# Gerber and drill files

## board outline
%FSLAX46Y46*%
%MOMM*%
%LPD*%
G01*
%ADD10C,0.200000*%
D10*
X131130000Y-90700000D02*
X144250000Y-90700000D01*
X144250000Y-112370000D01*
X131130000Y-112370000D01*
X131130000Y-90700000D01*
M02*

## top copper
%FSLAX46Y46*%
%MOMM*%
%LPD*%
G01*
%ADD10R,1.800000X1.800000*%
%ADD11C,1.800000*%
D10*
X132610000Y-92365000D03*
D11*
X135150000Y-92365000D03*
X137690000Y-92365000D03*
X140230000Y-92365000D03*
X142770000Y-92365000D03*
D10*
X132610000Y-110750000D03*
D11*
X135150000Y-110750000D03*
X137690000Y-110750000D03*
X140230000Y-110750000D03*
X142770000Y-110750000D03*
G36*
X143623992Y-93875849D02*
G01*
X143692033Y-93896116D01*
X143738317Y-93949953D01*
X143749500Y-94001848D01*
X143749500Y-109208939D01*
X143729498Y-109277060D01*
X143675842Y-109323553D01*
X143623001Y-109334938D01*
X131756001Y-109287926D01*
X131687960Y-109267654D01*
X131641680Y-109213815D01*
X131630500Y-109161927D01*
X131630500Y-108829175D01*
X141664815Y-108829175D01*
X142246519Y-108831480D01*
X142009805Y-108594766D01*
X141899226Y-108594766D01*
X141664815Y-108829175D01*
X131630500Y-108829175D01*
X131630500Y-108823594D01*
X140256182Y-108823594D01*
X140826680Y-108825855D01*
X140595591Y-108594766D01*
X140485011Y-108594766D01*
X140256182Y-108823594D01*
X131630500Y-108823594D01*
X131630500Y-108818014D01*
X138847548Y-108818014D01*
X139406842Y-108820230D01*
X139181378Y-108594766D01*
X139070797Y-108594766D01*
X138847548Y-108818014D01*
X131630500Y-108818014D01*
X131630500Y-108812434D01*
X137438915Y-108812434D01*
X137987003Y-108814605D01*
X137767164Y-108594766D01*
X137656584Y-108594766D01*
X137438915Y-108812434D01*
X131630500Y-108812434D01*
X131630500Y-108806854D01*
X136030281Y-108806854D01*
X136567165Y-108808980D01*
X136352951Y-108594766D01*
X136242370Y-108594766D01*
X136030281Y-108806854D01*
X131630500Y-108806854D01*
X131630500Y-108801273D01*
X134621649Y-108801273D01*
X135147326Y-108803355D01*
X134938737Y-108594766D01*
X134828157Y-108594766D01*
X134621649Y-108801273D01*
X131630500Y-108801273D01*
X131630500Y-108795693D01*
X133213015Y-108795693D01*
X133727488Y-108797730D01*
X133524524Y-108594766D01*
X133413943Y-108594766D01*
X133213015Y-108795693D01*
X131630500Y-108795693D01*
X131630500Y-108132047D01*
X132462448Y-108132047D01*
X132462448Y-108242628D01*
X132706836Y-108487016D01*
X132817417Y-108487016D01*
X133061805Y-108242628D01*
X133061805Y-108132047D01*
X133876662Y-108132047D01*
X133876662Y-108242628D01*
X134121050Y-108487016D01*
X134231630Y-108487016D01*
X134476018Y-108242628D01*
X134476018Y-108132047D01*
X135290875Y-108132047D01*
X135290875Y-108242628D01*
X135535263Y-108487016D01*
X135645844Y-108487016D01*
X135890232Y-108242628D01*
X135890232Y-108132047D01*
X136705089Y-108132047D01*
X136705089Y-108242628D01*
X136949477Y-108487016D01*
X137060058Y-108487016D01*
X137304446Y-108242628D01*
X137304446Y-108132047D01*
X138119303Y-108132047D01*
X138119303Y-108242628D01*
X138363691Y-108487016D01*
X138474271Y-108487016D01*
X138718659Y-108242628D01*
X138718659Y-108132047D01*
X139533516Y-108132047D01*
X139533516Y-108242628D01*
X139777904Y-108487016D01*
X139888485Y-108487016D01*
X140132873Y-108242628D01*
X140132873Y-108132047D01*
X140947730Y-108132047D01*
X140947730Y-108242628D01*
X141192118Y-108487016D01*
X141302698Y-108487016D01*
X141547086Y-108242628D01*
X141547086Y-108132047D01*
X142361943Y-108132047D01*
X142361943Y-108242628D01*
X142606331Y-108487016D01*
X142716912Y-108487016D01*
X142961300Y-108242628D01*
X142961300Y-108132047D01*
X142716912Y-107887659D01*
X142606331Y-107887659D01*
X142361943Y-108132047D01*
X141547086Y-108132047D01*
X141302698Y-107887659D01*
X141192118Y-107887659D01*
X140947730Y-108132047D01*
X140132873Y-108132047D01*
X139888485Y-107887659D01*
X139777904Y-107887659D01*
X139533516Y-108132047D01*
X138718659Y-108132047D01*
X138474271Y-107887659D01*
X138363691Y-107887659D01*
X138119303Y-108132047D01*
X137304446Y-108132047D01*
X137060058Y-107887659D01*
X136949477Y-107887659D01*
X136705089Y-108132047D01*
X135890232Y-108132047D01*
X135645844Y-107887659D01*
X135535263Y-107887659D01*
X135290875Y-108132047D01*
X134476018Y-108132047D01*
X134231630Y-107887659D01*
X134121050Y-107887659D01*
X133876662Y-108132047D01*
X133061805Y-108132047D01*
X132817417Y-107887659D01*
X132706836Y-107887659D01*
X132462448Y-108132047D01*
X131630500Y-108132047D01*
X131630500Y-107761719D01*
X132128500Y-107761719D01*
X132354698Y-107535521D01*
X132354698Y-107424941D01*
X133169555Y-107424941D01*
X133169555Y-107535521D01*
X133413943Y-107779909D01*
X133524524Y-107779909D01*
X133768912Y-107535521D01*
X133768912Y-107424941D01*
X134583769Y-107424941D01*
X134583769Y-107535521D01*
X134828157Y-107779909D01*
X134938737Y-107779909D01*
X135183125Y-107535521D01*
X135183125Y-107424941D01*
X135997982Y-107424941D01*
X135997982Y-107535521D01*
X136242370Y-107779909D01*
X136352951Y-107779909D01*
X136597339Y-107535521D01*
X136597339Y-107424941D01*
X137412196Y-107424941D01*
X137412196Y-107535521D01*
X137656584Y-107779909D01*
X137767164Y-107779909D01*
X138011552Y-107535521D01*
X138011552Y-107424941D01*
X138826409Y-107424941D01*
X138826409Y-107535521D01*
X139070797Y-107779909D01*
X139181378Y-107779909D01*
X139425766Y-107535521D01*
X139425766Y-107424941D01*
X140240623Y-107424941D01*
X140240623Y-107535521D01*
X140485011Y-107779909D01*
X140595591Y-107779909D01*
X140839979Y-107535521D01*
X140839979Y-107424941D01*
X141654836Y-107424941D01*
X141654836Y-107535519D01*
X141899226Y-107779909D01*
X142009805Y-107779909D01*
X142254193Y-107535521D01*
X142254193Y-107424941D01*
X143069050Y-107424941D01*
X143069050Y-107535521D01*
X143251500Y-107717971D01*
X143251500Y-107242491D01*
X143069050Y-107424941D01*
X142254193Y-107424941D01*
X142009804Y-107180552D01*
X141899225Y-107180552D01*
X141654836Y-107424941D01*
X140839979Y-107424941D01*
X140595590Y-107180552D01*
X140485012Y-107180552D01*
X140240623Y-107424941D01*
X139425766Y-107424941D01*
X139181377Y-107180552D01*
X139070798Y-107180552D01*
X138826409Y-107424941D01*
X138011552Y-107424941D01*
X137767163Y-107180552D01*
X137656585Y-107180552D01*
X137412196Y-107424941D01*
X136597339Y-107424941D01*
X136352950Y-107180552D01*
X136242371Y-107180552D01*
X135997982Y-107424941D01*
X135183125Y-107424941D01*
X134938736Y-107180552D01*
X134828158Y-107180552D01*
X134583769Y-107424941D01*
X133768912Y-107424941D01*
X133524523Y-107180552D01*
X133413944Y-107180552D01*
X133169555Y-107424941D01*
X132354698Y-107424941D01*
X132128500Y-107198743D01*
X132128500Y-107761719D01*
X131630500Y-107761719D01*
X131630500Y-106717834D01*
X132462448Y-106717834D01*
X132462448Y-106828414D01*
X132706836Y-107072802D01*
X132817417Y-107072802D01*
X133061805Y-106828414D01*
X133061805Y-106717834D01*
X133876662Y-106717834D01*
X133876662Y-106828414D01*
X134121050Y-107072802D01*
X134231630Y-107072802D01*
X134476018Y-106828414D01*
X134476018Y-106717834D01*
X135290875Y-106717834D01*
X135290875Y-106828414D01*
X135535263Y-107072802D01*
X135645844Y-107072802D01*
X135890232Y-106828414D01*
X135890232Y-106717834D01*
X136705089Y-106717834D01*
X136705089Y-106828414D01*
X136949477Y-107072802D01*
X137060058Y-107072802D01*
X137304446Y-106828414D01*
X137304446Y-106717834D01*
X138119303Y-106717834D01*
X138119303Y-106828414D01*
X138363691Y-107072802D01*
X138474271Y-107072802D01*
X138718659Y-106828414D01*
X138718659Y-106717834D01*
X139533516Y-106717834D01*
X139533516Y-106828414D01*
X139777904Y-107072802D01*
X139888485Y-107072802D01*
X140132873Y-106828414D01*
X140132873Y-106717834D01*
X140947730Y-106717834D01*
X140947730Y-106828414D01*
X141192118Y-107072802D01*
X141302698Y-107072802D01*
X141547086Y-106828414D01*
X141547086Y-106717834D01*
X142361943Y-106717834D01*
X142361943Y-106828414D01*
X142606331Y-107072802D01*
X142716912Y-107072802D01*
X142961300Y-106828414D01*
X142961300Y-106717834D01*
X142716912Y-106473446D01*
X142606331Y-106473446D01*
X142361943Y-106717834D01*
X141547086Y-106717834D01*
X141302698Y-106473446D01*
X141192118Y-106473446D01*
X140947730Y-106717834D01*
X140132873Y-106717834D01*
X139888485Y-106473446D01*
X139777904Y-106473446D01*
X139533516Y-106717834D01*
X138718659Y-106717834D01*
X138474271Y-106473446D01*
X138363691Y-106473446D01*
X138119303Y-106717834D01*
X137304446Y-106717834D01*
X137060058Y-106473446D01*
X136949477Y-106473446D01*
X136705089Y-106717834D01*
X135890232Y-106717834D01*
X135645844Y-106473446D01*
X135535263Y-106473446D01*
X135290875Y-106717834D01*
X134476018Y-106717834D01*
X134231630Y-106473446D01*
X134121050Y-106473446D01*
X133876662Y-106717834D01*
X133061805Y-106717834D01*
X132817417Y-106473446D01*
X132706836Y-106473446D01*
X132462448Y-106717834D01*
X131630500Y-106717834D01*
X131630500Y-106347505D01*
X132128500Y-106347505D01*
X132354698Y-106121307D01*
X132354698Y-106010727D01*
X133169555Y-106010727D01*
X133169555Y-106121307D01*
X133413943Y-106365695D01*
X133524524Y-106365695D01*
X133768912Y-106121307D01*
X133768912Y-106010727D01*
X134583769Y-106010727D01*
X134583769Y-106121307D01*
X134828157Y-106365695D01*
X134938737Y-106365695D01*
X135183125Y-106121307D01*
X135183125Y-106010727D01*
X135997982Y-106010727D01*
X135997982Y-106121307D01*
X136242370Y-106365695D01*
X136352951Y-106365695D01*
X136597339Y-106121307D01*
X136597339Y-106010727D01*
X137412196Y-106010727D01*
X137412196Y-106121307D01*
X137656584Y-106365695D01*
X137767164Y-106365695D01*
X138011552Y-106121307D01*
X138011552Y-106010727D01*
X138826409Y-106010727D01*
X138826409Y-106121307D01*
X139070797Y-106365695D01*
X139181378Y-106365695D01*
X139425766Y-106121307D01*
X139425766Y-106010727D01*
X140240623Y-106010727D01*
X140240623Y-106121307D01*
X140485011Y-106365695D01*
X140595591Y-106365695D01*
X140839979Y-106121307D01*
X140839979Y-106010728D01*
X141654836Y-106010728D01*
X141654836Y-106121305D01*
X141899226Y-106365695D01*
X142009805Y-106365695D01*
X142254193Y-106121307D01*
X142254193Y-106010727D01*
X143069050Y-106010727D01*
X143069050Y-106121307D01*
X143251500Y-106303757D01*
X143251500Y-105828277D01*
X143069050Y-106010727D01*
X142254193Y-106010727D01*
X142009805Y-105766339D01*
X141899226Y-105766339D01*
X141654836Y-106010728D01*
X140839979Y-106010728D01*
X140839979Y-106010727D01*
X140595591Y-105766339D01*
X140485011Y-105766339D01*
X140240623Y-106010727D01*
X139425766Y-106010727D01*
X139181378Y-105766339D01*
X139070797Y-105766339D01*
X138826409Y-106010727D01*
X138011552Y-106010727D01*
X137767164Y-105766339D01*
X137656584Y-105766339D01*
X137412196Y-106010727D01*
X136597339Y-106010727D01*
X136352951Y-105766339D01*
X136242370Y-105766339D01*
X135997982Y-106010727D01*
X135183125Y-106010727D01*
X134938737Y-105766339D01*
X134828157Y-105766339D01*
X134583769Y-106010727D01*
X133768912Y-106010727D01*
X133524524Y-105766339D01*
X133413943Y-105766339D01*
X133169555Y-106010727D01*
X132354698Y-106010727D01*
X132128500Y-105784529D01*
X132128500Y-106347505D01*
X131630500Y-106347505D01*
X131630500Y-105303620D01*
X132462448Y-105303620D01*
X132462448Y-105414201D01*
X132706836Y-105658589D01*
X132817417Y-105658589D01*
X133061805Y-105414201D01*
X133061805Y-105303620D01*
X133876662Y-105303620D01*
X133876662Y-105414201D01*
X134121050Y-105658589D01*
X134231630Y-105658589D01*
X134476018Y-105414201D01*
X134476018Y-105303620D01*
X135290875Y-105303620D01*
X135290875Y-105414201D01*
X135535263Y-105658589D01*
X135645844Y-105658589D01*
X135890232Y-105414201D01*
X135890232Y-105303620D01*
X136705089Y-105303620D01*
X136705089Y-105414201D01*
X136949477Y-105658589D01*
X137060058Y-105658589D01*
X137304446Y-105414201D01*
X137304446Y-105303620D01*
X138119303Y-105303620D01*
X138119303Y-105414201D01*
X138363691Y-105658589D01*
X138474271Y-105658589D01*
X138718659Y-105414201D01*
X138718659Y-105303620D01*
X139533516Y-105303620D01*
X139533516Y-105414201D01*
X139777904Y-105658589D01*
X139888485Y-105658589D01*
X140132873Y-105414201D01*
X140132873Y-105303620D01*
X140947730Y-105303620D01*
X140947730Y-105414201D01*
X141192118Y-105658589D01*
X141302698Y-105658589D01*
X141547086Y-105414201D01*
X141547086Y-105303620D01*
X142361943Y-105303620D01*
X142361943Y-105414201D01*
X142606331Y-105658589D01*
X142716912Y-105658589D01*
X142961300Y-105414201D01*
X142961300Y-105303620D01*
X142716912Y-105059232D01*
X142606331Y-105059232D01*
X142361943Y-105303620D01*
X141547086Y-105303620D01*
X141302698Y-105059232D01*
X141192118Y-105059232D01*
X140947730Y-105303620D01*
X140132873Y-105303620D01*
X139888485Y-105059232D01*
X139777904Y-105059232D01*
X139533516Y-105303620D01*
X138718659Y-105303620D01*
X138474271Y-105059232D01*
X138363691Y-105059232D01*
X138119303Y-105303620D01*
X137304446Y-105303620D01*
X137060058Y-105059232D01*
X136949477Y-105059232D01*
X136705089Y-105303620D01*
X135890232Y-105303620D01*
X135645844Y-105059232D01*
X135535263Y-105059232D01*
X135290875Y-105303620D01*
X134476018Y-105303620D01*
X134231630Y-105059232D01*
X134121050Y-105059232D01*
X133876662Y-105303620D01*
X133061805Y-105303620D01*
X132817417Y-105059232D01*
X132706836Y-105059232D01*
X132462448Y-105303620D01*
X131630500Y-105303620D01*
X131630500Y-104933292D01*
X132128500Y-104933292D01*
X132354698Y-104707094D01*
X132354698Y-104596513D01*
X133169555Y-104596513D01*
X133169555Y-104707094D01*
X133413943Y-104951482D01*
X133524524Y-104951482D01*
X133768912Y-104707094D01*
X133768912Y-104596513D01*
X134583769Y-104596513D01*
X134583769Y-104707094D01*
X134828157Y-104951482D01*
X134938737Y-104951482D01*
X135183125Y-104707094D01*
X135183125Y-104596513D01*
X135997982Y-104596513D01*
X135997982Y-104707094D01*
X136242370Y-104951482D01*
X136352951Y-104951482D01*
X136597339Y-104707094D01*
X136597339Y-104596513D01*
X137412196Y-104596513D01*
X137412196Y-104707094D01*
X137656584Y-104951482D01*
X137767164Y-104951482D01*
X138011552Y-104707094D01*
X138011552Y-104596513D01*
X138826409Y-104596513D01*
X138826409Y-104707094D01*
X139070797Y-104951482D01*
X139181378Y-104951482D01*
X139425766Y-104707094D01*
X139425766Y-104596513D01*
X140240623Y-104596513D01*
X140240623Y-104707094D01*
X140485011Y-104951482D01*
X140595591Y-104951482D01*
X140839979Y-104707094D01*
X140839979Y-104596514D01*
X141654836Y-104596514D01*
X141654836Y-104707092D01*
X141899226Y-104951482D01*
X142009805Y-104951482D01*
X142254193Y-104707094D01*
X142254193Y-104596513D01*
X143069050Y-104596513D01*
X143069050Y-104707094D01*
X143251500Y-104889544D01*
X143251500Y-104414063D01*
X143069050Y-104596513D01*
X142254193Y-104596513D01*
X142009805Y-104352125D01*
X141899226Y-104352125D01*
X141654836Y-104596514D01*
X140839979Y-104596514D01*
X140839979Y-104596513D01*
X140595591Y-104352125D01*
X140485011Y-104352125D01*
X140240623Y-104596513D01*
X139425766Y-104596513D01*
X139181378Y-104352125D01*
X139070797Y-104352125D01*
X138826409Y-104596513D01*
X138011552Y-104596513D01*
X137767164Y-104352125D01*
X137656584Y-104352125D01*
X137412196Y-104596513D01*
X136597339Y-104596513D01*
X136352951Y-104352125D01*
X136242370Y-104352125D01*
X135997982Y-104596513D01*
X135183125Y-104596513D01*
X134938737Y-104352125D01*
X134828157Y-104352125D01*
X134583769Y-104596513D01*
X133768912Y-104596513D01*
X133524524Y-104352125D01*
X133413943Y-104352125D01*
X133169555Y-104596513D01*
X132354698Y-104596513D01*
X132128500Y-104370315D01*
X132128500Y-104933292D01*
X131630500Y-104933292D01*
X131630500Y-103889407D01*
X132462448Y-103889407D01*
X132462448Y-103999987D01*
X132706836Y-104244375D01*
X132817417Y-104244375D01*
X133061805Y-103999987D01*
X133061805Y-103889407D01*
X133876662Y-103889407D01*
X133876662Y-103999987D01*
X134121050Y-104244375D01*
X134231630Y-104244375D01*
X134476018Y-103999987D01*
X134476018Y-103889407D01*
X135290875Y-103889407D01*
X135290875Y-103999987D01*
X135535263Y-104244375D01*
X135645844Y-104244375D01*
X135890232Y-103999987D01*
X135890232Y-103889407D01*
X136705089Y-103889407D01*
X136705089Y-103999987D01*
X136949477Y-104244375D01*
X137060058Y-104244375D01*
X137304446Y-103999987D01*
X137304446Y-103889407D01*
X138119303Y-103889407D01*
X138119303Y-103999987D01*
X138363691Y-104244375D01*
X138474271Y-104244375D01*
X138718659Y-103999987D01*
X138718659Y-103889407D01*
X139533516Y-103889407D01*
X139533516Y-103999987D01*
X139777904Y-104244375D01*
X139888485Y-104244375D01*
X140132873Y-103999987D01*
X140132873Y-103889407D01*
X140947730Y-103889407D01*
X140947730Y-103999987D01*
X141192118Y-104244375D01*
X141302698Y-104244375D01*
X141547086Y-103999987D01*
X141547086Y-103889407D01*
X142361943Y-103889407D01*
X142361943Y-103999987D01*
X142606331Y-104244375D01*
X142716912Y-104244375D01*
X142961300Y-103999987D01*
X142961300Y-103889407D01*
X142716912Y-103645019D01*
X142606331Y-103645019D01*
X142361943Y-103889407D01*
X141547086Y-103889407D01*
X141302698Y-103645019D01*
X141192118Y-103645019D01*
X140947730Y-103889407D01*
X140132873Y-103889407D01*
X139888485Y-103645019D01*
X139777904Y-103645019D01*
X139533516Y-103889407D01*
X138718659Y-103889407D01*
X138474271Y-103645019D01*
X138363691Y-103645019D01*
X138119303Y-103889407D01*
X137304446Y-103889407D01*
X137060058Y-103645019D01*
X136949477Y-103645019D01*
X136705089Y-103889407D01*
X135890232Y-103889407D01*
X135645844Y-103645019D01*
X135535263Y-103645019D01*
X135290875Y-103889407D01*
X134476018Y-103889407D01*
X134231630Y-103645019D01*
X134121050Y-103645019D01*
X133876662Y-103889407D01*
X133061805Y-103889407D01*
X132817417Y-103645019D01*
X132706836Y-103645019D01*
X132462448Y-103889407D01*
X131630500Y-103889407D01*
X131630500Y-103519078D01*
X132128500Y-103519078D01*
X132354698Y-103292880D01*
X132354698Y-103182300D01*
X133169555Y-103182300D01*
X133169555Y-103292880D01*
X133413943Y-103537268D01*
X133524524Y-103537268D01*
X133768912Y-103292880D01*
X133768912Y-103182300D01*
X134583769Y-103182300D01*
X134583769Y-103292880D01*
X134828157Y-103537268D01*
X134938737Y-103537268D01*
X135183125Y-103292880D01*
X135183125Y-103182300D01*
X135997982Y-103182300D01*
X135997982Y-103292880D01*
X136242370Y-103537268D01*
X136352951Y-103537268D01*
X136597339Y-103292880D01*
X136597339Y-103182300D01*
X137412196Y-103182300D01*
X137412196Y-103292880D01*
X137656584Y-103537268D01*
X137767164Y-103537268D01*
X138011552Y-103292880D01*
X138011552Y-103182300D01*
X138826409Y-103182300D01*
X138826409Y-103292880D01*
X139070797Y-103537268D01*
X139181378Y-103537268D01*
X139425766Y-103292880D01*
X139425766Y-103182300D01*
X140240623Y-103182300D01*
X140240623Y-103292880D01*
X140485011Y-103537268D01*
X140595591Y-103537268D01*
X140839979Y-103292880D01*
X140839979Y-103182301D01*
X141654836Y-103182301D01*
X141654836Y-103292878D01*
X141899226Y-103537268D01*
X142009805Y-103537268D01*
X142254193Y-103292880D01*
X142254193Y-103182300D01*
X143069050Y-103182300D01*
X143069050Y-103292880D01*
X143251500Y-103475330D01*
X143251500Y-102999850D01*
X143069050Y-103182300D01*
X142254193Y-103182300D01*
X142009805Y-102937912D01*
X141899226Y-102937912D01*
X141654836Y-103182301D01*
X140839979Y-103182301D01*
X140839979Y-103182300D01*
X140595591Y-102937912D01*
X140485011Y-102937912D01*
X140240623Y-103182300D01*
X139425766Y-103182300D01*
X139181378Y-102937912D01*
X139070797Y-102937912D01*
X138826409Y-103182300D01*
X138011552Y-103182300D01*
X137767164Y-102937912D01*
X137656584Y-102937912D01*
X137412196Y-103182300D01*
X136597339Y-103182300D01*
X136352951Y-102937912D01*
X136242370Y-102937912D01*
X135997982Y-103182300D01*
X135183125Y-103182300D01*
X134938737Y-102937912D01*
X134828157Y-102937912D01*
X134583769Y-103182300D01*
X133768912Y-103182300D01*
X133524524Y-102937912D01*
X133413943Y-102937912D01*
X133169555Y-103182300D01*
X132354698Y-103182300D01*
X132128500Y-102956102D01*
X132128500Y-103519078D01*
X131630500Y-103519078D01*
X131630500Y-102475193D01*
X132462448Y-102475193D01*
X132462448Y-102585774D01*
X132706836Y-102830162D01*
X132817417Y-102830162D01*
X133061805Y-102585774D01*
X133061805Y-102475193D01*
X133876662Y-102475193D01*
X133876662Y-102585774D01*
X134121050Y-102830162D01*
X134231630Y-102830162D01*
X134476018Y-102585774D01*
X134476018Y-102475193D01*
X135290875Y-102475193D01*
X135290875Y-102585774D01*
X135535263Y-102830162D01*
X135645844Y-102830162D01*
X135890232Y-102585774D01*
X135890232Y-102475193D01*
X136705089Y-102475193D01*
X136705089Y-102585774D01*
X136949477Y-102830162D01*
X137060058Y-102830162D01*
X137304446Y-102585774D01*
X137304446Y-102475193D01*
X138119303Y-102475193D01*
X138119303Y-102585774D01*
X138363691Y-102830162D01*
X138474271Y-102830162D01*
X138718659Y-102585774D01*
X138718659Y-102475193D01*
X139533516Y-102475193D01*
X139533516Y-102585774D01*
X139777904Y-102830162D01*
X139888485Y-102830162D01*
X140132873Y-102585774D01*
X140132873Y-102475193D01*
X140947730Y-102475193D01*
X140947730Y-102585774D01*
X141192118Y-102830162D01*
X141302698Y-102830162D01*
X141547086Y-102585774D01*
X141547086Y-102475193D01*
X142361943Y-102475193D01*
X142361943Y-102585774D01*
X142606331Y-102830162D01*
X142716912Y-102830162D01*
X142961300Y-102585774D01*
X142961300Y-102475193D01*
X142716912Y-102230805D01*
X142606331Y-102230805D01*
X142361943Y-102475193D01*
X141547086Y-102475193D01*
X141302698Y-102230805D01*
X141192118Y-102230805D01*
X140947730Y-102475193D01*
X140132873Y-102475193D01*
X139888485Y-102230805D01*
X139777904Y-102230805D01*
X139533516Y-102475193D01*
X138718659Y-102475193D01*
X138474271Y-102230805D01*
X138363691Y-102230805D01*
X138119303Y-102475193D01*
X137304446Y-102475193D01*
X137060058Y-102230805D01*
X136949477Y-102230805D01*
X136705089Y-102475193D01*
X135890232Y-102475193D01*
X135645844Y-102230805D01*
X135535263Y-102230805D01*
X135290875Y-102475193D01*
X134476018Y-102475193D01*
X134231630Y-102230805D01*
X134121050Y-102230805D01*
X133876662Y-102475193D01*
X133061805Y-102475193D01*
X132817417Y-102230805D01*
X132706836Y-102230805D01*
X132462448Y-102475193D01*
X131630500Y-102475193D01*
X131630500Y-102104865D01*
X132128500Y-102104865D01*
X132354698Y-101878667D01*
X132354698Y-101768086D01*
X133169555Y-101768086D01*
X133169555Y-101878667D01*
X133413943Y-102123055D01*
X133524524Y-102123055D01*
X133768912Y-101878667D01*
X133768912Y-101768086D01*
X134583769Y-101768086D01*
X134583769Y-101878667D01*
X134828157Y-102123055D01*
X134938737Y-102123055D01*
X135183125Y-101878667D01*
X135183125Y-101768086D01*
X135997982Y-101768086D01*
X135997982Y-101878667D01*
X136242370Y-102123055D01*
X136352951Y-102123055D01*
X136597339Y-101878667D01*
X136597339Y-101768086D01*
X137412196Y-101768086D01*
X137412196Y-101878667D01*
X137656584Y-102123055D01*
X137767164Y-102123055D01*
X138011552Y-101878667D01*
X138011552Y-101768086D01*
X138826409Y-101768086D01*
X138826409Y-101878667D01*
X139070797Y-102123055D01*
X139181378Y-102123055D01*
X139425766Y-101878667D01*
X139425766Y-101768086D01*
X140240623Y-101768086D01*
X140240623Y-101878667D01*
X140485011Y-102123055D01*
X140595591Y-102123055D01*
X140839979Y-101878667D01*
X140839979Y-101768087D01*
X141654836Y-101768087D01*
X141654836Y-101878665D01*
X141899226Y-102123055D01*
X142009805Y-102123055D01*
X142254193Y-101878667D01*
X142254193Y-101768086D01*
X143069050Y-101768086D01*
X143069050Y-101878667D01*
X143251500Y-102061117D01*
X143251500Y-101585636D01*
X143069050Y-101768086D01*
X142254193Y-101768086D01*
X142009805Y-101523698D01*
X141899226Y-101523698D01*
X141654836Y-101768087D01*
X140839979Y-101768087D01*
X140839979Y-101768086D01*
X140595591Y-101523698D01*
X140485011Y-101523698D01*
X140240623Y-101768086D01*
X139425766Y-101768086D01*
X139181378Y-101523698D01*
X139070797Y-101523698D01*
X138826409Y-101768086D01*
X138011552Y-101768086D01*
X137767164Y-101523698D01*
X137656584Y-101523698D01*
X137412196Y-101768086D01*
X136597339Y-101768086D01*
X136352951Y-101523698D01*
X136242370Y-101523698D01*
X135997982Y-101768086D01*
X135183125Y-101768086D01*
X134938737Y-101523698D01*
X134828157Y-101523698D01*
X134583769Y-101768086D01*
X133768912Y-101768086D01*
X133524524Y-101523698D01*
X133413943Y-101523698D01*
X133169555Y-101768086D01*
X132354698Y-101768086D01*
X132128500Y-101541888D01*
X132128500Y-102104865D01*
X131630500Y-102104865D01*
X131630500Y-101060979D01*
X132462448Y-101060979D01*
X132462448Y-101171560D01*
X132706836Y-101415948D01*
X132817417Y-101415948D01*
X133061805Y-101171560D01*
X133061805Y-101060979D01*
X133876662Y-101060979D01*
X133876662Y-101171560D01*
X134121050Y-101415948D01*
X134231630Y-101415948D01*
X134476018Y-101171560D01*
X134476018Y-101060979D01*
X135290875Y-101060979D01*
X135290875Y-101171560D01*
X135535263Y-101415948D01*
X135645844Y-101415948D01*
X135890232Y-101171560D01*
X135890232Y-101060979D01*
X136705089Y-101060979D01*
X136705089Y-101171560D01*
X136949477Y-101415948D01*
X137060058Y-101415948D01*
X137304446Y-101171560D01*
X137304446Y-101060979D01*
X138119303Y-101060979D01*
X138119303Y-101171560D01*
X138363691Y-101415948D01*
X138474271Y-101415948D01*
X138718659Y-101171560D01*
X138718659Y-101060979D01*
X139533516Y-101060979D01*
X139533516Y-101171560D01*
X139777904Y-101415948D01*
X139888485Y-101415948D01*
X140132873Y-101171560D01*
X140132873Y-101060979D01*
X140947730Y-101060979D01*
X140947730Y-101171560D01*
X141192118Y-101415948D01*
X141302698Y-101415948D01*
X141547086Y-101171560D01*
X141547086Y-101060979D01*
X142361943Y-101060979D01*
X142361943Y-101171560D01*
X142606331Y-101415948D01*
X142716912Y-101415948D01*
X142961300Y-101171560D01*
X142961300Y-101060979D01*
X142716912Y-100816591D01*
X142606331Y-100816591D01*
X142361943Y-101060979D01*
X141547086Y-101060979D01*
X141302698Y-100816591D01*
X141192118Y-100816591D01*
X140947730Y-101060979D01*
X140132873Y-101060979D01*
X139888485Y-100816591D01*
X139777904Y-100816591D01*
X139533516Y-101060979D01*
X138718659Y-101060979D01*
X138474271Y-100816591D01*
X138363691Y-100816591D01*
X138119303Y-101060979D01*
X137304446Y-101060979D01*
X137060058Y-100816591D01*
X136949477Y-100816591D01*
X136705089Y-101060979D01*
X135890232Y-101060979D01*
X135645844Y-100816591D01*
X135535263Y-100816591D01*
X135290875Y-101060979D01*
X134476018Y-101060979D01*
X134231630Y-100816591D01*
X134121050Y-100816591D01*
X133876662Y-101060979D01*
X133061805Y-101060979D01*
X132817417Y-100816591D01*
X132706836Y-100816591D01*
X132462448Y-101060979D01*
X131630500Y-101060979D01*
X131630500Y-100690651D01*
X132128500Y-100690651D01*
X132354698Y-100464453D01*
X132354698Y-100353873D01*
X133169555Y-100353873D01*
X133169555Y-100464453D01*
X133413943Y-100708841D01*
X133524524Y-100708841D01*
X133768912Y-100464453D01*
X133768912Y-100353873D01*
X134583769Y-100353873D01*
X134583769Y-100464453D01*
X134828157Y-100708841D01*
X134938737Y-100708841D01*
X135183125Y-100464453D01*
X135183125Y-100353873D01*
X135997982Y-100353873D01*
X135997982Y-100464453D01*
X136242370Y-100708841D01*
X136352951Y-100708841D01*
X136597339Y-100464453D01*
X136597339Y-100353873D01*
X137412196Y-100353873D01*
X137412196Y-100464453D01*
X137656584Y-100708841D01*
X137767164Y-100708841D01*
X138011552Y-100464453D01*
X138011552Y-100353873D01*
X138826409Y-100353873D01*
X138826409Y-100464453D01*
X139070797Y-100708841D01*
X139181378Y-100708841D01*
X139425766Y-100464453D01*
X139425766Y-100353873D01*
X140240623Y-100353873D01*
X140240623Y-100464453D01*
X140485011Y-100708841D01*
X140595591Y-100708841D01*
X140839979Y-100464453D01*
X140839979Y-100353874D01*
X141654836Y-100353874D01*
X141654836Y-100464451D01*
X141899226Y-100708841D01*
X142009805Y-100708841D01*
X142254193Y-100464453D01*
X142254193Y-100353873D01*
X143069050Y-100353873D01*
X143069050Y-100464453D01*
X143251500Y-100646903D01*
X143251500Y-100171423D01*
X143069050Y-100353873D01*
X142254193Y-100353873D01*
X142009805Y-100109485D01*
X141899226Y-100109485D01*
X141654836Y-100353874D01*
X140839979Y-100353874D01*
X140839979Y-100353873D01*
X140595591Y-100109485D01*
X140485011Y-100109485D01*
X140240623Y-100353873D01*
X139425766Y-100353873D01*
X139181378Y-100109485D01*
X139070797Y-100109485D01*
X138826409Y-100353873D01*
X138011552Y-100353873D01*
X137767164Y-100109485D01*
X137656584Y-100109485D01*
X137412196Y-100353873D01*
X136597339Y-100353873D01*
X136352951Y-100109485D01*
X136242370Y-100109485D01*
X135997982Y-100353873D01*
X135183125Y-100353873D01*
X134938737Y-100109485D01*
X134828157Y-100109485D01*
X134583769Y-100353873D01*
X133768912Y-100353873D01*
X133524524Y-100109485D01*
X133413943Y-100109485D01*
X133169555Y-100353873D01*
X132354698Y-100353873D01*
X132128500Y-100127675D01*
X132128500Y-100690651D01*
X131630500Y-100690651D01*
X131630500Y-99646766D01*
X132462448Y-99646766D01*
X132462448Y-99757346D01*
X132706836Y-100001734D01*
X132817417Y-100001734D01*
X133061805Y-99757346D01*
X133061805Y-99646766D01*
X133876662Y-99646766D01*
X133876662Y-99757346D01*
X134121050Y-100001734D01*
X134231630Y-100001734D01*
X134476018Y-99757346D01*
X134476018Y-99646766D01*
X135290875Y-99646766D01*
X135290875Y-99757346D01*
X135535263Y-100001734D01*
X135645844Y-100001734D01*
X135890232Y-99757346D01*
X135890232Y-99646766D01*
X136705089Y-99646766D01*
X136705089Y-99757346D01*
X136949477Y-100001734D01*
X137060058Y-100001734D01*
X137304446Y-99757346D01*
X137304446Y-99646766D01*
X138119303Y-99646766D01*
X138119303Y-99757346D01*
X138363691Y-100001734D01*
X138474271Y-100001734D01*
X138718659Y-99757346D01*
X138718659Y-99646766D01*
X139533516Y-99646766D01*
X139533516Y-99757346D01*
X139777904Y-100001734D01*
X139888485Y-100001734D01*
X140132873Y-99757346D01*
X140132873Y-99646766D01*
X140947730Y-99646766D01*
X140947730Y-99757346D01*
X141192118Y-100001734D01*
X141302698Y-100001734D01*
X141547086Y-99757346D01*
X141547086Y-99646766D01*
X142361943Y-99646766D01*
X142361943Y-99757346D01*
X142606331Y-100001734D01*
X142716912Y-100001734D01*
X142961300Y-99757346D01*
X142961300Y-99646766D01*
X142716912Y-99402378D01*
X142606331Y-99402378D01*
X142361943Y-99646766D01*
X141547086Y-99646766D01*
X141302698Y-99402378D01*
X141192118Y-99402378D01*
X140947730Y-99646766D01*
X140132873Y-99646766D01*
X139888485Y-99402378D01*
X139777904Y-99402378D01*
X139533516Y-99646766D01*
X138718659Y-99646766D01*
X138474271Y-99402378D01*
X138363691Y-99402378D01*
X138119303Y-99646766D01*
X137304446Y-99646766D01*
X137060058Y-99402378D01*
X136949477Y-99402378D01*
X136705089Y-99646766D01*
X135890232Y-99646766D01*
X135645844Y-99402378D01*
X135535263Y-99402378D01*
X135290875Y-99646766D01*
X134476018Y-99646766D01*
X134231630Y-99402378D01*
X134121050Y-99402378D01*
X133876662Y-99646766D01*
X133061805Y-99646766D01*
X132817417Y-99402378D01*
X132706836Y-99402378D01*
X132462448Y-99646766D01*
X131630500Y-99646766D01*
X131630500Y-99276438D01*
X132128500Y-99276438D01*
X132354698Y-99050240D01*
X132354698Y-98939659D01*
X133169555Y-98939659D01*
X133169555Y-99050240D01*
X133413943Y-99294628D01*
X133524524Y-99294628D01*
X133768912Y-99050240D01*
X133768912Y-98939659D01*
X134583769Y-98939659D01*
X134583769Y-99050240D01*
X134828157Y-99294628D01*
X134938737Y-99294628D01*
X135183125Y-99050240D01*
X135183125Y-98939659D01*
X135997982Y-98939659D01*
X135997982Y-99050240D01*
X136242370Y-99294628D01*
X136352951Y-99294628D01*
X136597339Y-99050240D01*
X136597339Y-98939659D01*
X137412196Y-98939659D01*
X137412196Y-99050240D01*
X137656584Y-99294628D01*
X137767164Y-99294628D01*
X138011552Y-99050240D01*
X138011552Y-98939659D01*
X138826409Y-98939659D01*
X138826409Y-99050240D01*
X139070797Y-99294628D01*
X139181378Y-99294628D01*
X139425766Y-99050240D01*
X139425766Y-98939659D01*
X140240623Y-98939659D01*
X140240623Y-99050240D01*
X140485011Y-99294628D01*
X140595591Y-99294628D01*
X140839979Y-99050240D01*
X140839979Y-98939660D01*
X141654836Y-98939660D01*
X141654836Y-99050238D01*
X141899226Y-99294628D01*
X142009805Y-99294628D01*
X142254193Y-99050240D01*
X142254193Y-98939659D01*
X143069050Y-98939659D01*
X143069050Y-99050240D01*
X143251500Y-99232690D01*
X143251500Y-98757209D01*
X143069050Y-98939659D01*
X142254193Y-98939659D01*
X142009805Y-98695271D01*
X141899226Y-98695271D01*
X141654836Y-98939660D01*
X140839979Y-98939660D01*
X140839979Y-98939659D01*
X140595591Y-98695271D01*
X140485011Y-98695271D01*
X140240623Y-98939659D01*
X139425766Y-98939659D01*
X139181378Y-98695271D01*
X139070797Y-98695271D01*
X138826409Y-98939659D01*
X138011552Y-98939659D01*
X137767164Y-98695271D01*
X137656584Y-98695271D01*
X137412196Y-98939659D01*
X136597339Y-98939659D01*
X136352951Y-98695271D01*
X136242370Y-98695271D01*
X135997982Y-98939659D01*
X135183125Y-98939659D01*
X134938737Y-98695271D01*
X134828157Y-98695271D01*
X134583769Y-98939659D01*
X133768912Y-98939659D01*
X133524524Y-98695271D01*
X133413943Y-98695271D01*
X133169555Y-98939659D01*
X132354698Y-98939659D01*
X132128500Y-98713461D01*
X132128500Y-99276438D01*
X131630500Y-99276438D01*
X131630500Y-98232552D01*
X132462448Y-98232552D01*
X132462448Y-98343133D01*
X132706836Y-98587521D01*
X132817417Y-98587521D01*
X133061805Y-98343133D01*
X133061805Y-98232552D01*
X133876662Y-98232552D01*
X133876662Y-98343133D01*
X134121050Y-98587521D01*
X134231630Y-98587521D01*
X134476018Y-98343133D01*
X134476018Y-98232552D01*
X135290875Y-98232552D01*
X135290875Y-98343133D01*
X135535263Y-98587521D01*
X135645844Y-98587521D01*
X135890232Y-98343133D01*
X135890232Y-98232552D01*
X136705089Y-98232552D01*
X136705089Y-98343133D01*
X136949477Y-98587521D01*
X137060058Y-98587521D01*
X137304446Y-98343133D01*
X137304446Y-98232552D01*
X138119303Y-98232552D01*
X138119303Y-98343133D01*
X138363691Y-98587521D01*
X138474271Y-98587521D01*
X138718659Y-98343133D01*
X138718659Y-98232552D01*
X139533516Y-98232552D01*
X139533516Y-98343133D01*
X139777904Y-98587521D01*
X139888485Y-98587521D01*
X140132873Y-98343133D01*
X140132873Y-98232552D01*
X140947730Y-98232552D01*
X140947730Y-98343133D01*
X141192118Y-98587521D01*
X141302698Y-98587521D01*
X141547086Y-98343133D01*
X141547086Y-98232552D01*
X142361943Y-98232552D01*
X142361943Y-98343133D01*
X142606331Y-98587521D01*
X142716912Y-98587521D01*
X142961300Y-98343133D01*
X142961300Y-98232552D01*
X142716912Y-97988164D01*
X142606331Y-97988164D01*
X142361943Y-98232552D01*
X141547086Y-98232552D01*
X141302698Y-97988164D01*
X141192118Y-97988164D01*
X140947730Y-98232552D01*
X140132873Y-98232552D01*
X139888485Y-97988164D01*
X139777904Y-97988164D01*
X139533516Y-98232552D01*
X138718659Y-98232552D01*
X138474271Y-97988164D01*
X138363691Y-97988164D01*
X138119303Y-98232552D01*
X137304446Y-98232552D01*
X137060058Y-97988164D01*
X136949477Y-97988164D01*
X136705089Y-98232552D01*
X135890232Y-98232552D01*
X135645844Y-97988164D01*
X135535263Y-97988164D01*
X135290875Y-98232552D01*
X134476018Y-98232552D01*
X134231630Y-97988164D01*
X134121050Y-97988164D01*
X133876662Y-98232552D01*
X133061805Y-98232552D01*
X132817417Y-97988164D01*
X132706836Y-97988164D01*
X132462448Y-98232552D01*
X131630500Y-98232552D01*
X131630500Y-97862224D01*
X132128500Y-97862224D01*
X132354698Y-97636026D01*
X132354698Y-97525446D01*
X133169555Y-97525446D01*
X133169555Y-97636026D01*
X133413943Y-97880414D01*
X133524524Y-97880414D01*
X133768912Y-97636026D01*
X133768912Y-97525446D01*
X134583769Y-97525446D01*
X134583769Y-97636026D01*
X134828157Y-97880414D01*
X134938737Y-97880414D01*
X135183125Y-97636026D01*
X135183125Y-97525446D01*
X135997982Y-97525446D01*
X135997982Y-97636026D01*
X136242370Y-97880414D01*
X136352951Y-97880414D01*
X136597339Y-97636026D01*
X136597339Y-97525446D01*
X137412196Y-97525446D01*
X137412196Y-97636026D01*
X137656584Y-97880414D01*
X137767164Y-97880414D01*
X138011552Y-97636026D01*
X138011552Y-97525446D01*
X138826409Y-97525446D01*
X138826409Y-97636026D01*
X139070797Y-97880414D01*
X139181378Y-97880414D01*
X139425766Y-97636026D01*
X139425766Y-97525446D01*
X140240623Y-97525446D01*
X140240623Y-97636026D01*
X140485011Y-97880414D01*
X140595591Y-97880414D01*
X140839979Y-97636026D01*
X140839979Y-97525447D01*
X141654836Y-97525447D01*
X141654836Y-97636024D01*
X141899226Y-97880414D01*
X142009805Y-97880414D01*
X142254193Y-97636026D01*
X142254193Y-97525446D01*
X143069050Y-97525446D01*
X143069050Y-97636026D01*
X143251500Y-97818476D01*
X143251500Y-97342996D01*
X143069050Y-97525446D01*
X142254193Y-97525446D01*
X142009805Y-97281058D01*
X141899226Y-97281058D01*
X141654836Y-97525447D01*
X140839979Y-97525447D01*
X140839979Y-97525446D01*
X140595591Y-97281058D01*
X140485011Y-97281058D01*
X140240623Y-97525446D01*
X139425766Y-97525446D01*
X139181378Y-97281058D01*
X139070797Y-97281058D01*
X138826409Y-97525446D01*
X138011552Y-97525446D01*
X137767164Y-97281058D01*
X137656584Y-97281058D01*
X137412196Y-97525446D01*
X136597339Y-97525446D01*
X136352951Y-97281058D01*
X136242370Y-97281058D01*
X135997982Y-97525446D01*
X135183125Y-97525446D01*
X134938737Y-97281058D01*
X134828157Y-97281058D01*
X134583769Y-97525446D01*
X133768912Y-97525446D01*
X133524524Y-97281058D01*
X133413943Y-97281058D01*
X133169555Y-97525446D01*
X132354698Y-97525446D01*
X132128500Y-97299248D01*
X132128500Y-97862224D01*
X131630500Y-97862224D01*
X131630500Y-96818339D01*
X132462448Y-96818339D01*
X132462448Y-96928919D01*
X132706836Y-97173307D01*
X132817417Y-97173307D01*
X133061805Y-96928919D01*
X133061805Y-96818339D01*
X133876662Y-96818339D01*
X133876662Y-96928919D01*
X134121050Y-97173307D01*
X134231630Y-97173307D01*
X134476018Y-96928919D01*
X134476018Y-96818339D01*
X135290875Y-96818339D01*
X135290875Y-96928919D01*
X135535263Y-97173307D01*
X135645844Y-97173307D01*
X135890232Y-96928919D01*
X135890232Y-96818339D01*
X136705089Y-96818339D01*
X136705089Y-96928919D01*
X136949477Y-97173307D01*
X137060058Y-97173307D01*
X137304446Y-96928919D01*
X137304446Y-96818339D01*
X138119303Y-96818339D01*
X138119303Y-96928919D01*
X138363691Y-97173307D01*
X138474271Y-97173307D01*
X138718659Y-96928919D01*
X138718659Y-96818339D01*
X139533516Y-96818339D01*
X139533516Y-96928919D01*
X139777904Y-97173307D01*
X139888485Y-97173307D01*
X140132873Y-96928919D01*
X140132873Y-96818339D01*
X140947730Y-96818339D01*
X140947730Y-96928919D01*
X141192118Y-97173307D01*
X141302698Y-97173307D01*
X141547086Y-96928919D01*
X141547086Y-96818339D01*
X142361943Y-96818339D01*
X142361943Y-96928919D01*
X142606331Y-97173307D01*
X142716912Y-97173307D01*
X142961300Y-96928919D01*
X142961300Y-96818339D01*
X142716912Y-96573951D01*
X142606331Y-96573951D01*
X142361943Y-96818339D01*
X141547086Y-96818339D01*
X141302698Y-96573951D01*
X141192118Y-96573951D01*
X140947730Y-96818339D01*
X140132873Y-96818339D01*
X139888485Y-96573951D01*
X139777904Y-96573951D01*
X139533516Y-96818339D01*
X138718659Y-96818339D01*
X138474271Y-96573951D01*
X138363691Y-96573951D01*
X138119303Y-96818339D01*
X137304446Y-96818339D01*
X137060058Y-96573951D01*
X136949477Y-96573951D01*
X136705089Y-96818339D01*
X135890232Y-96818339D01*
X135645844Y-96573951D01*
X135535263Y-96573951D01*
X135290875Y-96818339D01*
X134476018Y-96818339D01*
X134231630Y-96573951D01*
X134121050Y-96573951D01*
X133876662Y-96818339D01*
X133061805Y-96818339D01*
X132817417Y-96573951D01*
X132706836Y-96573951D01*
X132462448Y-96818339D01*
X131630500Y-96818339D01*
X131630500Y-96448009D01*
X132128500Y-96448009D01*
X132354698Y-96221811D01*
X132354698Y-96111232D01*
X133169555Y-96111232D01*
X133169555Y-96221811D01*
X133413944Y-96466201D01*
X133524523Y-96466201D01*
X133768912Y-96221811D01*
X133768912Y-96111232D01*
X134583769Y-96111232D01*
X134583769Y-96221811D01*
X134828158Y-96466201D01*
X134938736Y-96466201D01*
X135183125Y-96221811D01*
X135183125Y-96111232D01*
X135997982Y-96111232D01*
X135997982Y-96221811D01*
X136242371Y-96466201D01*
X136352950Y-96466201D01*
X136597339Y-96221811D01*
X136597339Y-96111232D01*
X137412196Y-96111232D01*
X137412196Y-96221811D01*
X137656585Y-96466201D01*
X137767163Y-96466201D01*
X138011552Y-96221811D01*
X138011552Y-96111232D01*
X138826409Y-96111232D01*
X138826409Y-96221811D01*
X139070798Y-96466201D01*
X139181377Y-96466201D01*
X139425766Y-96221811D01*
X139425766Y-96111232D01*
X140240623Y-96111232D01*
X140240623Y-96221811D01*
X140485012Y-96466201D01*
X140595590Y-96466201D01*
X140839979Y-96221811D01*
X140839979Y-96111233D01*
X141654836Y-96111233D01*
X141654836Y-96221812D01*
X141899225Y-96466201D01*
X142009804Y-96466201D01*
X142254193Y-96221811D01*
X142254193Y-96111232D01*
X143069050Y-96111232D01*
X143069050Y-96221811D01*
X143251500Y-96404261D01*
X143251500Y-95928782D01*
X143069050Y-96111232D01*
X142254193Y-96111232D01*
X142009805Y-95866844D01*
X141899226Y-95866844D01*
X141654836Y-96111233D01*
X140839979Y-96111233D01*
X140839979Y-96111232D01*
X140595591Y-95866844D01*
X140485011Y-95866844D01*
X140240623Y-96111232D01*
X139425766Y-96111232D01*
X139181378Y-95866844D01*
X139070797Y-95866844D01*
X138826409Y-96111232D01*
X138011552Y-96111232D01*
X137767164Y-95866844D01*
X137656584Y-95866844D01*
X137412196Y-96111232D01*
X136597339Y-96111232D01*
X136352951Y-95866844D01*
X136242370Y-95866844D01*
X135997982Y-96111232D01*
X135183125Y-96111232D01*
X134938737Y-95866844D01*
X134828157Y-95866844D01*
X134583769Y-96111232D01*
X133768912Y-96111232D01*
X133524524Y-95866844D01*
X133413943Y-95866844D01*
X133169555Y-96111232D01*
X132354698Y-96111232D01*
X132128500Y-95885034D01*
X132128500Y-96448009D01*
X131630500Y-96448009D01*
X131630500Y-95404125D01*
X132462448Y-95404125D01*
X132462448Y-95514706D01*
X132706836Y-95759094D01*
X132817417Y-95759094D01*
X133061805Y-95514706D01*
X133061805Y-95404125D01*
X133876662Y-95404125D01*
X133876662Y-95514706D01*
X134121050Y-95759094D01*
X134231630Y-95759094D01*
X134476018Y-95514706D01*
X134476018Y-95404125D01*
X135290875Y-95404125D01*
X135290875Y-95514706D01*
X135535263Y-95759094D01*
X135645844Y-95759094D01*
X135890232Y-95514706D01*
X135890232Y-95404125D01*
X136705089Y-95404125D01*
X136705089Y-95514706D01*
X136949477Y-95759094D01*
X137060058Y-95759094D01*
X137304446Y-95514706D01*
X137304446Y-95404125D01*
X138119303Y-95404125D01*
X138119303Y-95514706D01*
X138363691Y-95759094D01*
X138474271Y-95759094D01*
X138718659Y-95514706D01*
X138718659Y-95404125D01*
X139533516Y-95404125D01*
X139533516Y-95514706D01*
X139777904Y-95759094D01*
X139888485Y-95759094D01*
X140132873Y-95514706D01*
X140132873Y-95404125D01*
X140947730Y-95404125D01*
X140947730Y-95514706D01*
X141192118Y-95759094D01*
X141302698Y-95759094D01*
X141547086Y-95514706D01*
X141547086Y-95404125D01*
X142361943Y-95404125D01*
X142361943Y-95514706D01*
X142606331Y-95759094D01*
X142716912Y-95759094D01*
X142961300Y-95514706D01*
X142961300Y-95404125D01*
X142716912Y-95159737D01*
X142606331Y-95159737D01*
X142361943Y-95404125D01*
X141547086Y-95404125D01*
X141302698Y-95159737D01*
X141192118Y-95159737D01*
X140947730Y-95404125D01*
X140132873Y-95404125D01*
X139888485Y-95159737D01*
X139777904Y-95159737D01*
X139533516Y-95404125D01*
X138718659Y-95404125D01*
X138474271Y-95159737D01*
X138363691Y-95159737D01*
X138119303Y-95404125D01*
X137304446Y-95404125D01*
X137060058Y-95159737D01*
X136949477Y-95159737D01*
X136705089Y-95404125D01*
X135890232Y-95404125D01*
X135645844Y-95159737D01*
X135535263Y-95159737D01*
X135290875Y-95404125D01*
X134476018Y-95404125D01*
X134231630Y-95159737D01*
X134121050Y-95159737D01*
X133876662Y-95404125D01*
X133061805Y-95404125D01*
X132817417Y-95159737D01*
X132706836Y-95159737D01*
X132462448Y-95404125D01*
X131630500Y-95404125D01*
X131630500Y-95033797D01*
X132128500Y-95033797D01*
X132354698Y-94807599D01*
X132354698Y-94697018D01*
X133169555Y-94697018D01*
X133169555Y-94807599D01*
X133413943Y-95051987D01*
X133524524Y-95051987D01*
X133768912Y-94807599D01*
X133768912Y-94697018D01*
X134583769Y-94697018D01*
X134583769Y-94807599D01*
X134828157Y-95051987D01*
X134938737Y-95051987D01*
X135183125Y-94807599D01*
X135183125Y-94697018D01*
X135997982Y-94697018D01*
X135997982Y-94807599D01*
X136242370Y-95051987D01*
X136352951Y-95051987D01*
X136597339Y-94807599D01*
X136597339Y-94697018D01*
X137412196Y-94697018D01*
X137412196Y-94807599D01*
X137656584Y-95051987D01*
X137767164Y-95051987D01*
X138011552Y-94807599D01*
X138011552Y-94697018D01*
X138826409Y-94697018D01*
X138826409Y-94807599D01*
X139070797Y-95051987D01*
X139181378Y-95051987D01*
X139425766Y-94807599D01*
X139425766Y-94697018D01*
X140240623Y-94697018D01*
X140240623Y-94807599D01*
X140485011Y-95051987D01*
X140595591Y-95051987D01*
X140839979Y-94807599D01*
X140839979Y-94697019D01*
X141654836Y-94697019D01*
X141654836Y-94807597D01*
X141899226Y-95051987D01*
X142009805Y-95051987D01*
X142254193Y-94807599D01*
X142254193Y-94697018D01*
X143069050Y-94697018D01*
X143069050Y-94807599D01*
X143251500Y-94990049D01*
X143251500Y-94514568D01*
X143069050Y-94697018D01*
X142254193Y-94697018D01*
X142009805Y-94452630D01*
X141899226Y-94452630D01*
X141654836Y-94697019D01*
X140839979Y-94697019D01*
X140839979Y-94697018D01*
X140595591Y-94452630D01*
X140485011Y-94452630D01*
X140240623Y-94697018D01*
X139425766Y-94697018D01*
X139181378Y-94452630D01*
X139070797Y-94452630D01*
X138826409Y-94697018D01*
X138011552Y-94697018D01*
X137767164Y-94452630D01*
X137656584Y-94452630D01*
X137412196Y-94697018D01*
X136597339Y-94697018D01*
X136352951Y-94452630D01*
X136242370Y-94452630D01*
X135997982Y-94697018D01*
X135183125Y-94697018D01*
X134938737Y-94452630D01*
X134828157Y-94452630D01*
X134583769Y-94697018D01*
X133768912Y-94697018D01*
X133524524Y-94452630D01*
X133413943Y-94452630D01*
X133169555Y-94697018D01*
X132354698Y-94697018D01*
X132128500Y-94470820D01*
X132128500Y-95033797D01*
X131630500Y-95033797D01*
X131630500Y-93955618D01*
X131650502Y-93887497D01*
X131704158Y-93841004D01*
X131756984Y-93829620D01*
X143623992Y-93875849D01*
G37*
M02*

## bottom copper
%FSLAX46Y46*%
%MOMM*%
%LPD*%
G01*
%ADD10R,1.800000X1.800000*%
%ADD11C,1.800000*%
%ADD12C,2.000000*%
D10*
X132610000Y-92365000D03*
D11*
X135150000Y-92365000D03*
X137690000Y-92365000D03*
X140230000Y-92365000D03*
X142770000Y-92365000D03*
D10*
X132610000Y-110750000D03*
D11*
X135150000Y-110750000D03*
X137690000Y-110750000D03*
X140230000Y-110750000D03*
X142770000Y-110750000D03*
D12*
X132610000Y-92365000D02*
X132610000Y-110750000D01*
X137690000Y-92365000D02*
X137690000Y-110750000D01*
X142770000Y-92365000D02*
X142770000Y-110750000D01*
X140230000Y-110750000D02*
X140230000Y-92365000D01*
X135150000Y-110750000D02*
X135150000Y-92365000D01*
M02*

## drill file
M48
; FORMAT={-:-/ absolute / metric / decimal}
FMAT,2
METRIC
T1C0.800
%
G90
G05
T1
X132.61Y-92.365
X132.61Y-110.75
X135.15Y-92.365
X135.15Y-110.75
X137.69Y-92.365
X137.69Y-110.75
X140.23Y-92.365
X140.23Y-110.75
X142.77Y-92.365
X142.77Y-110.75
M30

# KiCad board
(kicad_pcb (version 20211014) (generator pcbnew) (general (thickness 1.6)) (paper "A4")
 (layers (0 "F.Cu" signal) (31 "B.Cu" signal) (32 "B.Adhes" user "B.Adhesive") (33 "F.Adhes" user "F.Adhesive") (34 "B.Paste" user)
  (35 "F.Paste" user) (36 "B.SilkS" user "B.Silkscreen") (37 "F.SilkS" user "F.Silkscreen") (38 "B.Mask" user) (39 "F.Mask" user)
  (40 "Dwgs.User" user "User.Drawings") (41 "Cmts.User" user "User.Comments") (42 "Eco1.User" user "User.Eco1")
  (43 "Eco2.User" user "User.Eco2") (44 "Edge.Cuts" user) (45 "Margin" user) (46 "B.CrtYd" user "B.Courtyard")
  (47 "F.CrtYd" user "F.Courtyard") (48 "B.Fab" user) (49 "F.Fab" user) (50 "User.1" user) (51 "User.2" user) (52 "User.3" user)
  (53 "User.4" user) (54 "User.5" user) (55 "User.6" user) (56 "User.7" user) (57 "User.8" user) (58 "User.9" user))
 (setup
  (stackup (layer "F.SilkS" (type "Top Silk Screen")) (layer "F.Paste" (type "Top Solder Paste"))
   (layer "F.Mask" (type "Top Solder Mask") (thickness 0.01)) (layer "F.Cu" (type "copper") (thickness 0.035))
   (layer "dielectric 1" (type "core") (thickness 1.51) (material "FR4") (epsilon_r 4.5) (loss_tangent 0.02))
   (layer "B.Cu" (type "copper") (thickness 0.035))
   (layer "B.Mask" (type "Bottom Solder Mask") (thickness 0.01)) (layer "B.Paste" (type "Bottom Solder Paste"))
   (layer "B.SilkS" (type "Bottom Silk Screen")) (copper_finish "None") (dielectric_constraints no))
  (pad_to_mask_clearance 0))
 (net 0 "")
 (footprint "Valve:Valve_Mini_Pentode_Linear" (layer "F.Cu") (at 132.61 92.365)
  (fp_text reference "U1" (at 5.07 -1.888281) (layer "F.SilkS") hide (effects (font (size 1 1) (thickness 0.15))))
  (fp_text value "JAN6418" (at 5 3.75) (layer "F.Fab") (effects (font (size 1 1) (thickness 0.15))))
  (pad "1" thru_hole rect (at 0 0) (size 1.8 1.8) (drill 0.8) (layers *.Cu *.Mask))
  (pad "2" thru_hole circle (at 2.54 0) (size 1.8 1.8) (drill 0.8) (layers *.Cu *.Mask))
  (pad "3" thru_hole circle (at 5.08 0) (size 1.8 1.8) (drill 0.8) (layers *.Cu *.Mask))
  (pad "4" thru_hole circle (at 7.62 0) (size 1.8 1.8) (drill 0.8) (layers *.Cu *.Mask))
  (pad "5" thru_hole circle (at 10.16 0) (size 1.8 1.8) (drill 0.8) (layers *.Cu *.Mask)))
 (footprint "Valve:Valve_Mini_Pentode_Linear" (layer "F.Cu") (at 132.61 110.75)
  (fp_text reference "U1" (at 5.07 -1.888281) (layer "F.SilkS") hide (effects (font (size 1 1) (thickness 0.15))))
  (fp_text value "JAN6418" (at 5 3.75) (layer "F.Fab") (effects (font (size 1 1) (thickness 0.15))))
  (pad "1" thru_hole rect (at 0 0) (size 1.8 1.8) (drill 0.8) (layers *.Cu *.Mask))
  (pad "2" thru_hole circle (at 2.54 0) (size 1.8 1.8) (drill 0.8) (layers *.Cu *.Mask))
  (pad "3" thru_hole circle (at 5.08 0) (size 1.8 1.8) (drill 0.8) (layers *.Cu *.Mask))
  (pad "4" thru_hole circle (at 7.62 0) (size 1.8 1.8) (drill 0.8) (layers *.Cu *.Mask))
  (pad "5" thru_hole circle (at 10.16 0) (size 1.8 1.8) (drill 0.8) (layers *.Cu *.Mask)))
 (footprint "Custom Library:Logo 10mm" (layer "F.Cu") (at 137.69 101.530068)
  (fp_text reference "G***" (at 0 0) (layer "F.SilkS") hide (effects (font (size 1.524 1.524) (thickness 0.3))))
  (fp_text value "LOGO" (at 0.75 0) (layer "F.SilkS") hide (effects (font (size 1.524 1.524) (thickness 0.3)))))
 (gr_rect (start 131.13 90.7) (end 144.25 112.37) (layer "Edge.Cuts") (width 0.2) (fill none))
 (segment (start 132.61 92.365) (end 132.61 110.75) (width 2) (layer "B.Cu") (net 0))
 (segment (start 137.69 92.365) (end 137.69 110.75) (width 2) (layer "B.Cu") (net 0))
 (segment (start 142.77 92.365) (end 142.77 110.75) (width 2) (layer "B.Cu") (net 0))
 (segment (start 140.23 110.75) (end 140.23 92.365) (width 2) (layer "B.Cu") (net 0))
 (segment (start 135.15 110.75) (end 135.15 92.365) (width 2) (layer "B.Cu") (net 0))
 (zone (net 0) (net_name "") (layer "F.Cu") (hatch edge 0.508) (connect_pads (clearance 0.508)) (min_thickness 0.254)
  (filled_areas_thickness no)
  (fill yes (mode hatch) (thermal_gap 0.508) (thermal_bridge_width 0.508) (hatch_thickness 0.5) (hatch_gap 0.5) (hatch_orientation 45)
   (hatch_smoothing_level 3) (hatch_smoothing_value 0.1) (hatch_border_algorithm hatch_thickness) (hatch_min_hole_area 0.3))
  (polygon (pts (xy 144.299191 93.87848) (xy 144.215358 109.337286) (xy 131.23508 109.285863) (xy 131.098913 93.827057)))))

